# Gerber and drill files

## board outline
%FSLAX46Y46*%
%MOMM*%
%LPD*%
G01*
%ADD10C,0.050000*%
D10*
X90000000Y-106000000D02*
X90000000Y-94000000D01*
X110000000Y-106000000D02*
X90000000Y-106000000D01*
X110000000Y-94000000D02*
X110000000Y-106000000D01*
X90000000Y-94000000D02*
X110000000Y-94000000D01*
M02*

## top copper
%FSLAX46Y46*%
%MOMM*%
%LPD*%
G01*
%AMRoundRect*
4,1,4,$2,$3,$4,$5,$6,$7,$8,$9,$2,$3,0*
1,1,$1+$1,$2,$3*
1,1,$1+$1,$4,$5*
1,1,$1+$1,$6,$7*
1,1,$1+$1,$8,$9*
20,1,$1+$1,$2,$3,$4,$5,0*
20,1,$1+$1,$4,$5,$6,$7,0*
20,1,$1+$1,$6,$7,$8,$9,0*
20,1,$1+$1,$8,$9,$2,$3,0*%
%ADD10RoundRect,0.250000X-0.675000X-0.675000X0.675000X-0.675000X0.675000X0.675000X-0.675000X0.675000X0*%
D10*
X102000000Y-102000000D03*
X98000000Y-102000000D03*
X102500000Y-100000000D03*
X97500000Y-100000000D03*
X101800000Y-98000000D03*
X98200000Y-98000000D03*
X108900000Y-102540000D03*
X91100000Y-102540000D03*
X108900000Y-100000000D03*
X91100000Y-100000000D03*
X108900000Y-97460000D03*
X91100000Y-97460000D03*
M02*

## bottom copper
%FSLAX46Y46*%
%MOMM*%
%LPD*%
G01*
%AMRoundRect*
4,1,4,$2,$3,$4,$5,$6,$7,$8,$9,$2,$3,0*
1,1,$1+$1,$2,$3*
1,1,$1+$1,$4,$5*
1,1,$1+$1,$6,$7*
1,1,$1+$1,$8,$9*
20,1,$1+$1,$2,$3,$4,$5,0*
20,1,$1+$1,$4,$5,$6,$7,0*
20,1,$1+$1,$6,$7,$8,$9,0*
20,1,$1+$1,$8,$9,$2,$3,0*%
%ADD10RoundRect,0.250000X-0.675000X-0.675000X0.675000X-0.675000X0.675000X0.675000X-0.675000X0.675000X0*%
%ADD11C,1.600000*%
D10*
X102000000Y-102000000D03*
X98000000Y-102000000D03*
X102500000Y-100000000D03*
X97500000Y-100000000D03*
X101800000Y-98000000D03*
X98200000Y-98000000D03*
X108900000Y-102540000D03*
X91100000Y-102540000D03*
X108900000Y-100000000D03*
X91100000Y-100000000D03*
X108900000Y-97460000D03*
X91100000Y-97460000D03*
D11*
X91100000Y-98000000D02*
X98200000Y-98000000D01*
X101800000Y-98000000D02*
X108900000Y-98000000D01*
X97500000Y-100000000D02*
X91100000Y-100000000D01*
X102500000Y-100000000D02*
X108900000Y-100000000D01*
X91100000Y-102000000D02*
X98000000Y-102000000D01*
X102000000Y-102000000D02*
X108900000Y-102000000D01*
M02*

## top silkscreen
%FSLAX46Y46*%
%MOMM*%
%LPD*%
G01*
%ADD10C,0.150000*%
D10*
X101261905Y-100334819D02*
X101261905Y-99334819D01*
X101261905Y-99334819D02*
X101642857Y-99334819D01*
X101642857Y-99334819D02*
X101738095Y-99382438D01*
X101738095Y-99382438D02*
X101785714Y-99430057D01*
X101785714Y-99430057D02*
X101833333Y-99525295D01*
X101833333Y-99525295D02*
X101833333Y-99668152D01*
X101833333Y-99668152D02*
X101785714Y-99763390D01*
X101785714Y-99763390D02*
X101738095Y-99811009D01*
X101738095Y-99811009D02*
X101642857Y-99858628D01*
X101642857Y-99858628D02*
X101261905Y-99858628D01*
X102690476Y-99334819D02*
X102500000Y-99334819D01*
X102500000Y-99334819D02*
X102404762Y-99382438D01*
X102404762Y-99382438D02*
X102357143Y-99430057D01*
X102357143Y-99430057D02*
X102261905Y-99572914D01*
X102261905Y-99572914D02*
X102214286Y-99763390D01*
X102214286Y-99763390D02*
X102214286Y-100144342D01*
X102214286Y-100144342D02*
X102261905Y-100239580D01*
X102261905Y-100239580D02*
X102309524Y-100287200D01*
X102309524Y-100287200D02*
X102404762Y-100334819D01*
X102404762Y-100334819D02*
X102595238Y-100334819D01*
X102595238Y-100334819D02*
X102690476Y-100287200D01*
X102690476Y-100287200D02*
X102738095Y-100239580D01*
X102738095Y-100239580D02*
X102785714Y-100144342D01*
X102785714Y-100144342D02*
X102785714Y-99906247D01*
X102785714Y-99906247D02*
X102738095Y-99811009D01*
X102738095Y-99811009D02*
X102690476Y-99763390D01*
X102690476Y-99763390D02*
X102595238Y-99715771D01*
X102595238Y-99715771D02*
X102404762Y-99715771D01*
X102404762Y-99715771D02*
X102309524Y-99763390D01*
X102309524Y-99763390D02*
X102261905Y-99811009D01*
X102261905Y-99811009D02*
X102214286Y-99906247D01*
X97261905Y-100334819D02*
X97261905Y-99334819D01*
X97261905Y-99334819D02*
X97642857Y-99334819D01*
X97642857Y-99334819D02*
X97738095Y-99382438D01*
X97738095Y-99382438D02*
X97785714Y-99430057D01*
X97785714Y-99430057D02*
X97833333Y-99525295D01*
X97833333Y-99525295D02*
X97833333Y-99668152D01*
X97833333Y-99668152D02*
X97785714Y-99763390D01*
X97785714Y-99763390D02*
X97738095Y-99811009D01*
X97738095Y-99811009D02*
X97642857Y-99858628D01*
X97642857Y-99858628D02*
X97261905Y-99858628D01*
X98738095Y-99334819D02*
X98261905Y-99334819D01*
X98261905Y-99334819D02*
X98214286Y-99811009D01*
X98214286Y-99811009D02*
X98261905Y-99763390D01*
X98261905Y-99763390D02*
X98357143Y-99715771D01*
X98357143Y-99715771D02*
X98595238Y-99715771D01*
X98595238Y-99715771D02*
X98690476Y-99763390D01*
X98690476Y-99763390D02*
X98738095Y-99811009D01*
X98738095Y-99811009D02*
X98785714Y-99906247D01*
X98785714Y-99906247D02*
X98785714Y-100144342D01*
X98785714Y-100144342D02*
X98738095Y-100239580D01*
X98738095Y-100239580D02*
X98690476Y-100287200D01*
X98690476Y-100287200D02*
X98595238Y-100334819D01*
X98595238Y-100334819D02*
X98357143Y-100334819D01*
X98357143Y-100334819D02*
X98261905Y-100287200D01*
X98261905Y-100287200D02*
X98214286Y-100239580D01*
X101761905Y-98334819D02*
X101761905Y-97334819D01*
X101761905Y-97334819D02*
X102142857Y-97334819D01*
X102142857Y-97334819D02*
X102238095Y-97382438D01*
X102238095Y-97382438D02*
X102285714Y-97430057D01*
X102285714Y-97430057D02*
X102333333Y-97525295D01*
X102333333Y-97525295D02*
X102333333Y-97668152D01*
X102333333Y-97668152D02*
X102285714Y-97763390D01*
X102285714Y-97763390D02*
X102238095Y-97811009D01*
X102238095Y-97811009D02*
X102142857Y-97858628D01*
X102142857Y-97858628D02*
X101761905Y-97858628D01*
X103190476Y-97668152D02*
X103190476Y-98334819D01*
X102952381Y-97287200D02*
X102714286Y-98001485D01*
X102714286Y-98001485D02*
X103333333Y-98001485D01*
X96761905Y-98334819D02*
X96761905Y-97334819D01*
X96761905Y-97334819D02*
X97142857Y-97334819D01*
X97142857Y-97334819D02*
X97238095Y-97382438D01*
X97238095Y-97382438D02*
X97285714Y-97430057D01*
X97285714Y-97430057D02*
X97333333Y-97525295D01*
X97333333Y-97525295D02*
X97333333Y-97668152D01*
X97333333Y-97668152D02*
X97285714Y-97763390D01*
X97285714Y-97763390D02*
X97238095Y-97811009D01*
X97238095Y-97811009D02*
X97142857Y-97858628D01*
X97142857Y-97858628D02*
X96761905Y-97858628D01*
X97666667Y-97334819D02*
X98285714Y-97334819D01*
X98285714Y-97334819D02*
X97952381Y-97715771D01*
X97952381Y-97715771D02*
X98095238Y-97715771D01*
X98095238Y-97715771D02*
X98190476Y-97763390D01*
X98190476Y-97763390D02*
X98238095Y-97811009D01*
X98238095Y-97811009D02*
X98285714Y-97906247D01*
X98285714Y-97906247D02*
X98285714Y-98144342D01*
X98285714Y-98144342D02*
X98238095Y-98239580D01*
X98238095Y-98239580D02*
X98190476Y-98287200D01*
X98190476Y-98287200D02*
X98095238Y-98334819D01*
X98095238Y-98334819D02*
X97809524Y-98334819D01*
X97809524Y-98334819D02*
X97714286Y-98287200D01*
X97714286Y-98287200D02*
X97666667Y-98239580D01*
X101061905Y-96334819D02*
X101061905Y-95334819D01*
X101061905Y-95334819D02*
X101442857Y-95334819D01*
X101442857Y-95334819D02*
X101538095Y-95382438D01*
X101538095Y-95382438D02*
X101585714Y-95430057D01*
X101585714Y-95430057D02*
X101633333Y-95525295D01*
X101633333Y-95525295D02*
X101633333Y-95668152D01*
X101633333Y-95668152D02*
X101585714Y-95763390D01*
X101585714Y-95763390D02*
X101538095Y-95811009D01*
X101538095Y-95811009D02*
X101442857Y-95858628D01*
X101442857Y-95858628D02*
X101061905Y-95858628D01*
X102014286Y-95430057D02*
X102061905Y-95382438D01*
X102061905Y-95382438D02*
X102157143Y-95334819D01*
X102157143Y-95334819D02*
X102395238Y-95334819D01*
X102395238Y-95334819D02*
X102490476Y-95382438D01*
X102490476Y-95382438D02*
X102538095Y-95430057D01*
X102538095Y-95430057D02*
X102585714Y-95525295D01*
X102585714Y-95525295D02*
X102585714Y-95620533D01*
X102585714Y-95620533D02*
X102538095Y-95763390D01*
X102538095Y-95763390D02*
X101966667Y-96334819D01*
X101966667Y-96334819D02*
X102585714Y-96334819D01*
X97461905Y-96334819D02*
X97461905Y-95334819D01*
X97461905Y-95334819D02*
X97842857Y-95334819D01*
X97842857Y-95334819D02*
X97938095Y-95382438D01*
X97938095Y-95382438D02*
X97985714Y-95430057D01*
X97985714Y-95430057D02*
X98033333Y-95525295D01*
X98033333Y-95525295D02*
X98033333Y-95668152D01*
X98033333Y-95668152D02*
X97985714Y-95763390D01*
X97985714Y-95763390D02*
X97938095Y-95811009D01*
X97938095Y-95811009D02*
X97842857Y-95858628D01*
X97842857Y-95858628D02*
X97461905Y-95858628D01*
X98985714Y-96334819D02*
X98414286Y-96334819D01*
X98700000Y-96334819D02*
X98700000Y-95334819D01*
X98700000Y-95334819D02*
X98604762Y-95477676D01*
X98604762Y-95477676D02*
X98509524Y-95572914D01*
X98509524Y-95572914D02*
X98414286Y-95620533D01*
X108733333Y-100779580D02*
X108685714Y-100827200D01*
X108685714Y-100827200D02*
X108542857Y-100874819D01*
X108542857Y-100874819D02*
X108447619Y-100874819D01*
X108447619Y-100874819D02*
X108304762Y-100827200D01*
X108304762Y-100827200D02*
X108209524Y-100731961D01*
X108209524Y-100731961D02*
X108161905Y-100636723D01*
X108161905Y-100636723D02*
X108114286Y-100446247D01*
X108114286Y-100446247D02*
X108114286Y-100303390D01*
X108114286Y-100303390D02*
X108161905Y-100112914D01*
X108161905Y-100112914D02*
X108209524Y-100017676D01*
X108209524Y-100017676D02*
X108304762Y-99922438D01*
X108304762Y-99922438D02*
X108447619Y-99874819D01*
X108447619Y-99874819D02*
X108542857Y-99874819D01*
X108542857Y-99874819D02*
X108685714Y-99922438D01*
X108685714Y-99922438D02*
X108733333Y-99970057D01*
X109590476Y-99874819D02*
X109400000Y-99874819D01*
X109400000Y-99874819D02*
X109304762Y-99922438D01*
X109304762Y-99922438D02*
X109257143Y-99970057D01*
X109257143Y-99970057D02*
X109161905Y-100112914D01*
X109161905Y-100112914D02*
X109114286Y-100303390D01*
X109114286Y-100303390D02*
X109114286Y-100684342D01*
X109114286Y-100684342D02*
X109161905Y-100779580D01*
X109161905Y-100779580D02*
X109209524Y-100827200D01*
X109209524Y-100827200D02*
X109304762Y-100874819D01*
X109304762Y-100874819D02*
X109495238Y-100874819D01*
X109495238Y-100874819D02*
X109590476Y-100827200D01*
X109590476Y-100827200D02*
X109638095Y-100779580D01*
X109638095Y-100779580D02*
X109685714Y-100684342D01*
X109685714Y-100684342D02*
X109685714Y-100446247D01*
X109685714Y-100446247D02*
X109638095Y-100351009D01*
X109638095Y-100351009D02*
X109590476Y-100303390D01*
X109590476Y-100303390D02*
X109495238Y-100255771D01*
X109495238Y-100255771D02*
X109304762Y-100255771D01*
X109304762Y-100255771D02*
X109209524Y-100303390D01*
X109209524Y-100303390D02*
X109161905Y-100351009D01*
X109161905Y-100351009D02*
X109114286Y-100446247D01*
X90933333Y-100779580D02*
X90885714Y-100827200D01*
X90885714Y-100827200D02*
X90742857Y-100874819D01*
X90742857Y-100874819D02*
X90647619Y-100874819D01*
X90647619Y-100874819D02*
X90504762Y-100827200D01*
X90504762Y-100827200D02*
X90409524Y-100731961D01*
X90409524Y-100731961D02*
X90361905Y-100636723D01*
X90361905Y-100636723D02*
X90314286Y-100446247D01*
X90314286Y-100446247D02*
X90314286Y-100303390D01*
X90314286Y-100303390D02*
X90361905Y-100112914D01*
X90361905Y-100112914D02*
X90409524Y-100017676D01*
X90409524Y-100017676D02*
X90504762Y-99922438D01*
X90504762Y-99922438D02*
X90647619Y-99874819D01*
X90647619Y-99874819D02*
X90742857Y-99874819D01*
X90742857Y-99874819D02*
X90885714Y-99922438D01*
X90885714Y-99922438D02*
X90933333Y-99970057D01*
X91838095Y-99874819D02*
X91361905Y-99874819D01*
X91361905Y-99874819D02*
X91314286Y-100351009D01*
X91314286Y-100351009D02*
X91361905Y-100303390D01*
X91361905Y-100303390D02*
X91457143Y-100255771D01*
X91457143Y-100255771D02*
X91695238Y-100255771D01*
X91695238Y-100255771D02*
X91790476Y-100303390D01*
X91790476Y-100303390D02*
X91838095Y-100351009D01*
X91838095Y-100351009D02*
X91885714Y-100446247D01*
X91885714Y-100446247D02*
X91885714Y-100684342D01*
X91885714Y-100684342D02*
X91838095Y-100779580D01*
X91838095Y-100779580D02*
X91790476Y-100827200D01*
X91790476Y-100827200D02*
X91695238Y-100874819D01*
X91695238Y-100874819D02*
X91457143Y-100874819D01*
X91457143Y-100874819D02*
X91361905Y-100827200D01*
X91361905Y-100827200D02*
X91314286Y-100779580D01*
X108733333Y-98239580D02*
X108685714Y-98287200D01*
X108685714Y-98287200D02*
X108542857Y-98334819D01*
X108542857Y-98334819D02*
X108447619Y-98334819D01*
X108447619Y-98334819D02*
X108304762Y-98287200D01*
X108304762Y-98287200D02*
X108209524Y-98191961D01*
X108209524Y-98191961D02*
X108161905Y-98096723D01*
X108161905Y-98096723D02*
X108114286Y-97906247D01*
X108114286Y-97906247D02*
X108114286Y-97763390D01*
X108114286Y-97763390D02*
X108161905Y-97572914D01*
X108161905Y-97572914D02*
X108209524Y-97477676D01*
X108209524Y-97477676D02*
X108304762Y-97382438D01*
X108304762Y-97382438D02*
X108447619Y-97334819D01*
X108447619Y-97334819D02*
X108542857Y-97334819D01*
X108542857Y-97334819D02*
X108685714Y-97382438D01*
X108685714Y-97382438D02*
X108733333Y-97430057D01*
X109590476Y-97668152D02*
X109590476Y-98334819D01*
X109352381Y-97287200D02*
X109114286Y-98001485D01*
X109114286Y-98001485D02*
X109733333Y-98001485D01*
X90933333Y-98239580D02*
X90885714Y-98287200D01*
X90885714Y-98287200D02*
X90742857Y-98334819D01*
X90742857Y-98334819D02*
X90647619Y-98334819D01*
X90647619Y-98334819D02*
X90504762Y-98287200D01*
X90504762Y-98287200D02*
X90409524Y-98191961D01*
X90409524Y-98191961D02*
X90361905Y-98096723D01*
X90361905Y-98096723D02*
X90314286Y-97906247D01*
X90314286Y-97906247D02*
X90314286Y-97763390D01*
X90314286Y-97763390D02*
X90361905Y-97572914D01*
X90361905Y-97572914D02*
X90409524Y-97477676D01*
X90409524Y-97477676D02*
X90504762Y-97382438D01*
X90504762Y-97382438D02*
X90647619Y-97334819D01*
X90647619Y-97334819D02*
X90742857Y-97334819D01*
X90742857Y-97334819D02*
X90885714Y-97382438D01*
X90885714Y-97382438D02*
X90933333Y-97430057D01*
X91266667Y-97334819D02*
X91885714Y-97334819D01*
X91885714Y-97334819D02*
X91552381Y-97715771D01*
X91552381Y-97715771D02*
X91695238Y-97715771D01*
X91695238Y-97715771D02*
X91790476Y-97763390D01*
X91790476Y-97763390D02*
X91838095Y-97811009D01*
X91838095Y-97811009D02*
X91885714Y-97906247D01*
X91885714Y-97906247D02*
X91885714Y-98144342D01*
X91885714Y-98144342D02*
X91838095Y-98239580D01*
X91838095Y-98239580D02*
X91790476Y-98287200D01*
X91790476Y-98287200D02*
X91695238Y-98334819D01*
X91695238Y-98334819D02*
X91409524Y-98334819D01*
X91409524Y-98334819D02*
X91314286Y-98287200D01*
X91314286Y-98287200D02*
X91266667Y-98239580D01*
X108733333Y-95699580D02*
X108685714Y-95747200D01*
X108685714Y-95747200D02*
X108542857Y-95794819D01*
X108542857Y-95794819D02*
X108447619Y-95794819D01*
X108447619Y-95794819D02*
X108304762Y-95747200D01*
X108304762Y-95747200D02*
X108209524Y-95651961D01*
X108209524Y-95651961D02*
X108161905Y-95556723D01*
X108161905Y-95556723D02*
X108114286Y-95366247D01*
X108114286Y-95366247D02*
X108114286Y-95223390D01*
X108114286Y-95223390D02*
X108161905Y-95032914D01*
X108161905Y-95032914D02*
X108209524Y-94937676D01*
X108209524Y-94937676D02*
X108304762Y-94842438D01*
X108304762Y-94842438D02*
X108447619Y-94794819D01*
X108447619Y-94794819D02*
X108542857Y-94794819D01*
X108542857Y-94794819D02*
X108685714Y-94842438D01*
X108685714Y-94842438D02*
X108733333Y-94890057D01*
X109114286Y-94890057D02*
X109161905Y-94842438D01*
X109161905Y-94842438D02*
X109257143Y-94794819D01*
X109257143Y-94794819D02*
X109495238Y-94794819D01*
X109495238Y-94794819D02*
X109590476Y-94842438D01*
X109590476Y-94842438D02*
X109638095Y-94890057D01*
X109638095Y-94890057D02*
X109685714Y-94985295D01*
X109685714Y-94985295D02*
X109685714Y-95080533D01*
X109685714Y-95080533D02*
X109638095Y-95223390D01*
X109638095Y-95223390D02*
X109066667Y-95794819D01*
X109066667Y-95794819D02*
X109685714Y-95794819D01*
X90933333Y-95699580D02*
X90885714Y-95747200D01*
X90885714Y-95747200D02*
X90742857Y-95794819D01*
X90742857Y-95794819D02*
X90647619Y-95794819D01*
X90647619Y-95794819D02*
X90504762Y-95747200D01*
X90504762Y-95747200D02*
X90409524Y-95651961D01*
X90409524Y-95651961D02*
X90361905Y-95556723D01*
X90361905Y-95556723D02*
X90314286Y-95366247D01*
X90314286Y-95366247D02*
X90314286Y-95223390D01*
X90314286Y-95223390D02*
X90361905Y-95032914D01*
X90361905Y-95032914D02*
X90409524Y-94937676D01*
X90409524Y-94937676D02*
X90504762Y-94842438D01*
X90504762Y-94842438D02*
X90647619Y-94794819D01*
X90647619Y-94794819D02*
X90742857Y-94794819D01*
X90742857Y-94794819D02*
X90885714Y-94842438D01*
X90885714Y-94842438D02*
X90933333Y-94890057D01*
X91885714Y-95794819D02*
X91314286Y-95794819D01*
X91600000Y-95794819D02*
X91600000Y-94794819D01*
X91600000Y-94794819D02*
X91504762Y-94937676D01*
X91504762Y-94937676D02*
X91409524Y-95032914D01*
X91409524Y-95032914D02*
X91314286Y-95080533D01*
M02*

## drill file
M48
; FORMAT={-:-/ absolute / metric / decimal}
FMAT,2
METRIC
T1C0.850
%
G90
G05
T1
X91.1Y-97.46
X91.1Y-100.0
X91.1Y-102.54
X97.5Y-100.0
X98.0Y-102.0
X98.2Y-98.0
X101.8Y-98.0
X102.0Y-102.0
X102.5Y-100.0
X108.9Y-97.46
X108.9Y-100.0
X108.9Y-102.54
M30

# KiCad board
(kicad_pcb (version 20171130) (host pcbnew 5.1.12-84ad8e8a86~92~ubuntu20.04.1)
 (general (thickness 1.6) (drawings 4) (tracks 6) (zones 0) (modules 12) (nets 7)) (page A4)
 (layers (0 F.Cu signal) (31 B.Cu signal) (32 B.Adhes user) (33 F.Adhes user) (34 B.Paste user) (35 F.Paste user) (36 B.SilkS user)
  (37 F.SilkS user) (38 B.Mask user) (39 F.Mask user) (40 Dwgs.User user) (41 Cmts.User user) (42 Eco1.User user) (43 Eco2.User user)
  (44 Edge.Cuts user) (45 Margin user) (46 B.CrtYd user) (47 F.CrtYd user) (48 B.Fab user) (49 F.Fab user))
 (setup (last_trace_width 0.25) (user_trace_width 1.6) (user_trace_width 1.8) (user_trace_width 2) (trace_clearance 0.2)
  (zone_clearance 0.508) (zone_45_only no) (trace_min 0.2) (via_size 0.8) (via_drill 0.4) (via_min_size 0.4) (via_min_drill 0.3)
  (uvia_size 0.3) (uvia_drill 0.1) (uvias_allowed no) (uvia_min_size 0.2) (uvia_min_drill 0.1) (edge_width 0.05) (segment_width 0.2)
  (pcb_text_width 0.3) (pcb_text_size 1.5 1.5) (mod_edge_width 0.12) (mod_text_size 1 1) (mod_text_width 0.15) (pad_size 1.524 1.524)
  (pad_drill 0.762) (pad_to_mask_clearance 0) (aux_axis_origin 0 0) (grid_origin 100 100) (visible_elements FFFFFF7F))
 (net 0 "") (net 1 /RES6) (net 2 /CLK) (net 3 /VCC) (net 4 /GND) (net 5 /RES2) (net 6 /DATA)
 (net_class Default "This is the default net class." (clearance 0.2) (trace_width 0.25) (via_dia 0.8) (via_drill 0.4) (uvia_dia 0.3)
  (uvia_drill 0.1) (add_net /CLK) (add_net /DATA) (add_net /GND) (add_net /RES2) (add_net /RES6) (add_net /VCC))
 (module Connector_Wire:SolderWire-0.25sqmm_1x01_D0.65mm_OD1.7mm (layer F.Cu) (at 102 102)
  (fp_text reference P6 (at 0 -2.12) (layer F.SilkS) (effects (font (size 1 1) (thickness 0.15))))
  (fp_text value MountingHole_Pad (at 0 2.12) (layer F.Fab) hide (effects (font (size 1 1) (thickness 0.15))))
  (pad 1 thru_hole roundrect (at 0 0) (size 1.85 1.85) (drill 0.85) (layers *.Cu *.Mask) (roundrect_rratio 0.135135) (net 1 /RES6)))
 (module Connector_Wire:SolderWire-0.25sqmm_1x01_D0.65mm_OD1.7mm (layer F.Cu) (at 98 102)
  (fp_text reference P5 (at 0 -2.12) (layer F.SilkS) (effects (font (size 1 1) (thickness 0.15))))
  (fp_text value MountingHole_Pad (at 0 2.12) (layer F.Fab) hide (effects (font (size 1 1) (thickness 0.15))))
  (pad 1 thru_hole roundrect (at 0 0) (size 1.85 1.85) (drill 0.85) (layers *.Cu *.Mask) (roundrect_rratio 0.135135) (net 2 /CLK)))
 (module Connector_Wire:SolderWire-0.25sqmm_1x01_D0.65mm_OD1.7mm (layer F.Cu) (at 102.5 100)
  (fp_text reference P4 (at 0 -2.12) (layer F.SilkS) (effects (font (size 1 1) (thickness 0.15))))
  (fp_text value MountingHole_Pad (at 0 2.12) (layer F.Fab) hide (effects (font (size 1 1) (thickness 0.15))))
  (pad 1 thru_hole roundrect (at 0 0) (size 1.85 1.85) (drill 0.85) (layers *.Cu *.Mask) (roundrect_rratio 0.135135) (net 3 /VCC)))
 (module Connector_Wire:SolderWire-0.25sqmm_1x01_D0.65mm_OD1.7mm (layer F.Cu) (at 97.5 100)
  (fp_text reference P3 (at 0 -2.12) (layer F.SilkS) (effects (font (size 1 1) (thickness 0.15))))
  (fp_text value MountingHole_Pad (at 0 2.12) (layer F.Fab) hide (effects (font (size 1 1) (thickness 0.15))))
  (pad 1 thru_hole roundrect (at 0 0) (size 1.85 1.85) (drill 0.85) (layers *.Cu *.Mask) (roundrect_rratio 0.135135) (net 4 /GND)))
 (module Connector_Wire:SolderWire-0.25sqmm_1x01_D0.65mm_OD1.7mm (layer F.Cu) (at 101.8 98)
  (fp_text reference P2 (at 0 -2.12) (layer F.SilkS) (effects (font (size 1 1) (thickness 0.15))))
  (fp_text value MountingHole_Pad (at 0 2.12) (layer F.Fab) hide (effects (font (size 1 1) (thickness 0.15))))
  (pad 1 thru_hole roundrect (at 0 0) (size 1.85 1.85) (drill 0.85) (layers *.Cu *.Mask) (roundrect_rratio 0.135135) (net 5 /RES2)))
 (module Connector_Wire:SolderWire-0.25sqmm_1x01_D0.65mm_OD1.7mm (layer F.Cu) (at 98.2 98)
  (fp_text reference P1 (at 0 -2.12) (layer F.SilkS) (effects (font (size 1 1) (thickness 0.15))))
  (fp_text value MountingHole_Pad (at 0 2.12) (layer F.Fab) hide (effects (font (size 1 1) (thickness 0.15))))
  (pad 1 thru_hole roundrect (at 0 0) (size 1.85 1.85) (drill 0.85) (layers *.Cu *.Mask) (roundrect_rratio 0.135135) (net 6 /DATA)))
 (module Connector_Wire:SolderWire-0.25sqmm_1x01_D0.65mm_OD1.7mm (layer F.Cu) (at 108.9 102.54)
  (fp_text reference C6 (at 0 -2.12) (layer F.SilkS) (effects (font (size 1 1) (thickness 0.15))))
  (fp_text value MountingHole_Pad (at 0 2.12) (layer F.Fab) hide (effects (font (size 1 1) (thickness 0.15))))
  (pad 1 thru_hole roundrect (at 0 0) (size 1.85 1.85) (drill 0.85) (layers *.Cu *.Mask) (roundrect_rratio 0.135135) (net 1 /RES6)))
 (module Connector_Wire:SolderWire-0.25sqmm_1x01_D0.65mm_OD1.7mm (layer F.Cu) (at 91.1 102.54)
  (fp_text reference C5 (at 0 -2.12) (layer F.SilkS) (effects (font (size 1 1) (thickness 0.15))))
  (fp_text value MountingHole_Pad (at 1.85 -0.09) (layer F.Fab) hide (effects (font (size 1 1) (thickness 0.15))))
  (pad 1 thru_hole roundrect (at 0 0) (size 1.85 1.85) (drill 0.85) (layers *.Cu *.Mask) (roundrect_rratio 0.135135) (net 2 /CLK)))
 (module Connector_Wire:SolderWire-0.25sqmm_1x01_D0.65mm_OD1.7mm (layer F.Cu) (at 108.9 100)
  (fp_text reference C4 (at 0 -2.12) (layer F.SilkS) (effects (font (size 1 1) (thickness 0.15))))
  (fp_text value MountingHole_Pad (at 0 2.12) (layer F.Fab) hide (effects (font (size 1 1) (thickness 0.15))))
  (pad 1 thru_hole roundrect (at 0 0) (size 1.85 1.85) (drill 0.85) (layers *.Cu *.Mask) (roundrect_rratio 0.135135) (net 3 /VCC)))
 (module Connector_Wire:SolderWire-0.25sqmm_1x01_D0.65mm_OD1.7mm (layer F.Cu) (at 91.1 100)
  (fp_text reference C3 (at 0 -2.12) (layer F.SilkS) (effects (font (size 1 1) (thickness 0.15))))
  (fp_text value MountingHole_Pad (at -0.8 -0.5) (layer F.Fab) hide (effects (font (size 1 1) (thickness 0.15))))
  (pad 1 thru_hole roundrect (at 0 0) (size 1.85 1.85) (drill 0.85) (layers *.Cu *.Mask) (roundrect_rratio 0.135135) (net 4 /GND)))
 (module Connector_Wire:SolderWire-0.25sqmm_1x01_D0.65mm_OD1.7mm (layer F.Cu) (at 108.9 97.46)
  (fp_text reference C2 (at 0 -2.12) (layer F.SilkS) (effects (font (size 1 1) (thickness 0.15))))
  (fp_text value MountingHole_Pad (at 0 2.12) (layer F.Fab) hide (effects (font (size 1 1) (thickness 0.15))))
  (pad 1 thru_hole roundrect (at 0 0) (size 1.85 1.85) (drill 0.85) (layers *.Cu *.Mask) (roundrect_rratio 0.135135) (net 5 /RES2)))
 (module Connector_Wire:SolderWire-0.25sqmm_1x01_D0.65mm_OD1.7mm (layer F.Cu) (at 91.1 97.46)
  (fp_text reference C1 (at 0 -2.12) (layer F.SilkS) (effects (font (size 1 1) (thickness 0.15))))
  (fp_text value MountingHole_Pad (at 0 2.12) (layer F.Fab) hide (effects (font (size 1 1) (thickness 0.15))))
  (pad 1 thru_hole roundrect (at 0 0) (size 1.85 1.85) (drill 0.85) (layers *.Cu *.Mask) (roundrect_rratio 0.135135) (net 6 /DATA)))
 (gr_line (start 90 106) (end 90 94) (layer Edge.Cuts) (width 0.05))
 (gr_line (start 110 106) (end 90 106) (layer Edge.Cuts) (width 0.05))
 (gr_line (start 110 94) (end 110 106) (layer Edge.Cuts) (width 0.05))
 (gr_line (start 90 94) (end 110 94) (layer Edge.Cuts) (width 0.05))
 (segment (start 91.1 98) (end 98.2 98) (width 1.6) (layer B.Cu) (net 6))
 (segment (start 101.8 98) (end 108.9 98) (width 1.6) (layer B.Cu) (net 5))
 (segment (start 97.5 100) (end 91.1 100) (width 1.6) (layer B.Cu) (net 4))
 (segment (start 102.5 100) (end 108.9 100) (width 1.6) (layer B.Cu) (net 3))
 (segment (start 91.1 102) (end 98 102) (width 1.6) (layer B.Cu) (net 2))
 (segment (start 102 102) (end 108.9 102) (width 1.6) (layer B.Cu) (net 1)))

